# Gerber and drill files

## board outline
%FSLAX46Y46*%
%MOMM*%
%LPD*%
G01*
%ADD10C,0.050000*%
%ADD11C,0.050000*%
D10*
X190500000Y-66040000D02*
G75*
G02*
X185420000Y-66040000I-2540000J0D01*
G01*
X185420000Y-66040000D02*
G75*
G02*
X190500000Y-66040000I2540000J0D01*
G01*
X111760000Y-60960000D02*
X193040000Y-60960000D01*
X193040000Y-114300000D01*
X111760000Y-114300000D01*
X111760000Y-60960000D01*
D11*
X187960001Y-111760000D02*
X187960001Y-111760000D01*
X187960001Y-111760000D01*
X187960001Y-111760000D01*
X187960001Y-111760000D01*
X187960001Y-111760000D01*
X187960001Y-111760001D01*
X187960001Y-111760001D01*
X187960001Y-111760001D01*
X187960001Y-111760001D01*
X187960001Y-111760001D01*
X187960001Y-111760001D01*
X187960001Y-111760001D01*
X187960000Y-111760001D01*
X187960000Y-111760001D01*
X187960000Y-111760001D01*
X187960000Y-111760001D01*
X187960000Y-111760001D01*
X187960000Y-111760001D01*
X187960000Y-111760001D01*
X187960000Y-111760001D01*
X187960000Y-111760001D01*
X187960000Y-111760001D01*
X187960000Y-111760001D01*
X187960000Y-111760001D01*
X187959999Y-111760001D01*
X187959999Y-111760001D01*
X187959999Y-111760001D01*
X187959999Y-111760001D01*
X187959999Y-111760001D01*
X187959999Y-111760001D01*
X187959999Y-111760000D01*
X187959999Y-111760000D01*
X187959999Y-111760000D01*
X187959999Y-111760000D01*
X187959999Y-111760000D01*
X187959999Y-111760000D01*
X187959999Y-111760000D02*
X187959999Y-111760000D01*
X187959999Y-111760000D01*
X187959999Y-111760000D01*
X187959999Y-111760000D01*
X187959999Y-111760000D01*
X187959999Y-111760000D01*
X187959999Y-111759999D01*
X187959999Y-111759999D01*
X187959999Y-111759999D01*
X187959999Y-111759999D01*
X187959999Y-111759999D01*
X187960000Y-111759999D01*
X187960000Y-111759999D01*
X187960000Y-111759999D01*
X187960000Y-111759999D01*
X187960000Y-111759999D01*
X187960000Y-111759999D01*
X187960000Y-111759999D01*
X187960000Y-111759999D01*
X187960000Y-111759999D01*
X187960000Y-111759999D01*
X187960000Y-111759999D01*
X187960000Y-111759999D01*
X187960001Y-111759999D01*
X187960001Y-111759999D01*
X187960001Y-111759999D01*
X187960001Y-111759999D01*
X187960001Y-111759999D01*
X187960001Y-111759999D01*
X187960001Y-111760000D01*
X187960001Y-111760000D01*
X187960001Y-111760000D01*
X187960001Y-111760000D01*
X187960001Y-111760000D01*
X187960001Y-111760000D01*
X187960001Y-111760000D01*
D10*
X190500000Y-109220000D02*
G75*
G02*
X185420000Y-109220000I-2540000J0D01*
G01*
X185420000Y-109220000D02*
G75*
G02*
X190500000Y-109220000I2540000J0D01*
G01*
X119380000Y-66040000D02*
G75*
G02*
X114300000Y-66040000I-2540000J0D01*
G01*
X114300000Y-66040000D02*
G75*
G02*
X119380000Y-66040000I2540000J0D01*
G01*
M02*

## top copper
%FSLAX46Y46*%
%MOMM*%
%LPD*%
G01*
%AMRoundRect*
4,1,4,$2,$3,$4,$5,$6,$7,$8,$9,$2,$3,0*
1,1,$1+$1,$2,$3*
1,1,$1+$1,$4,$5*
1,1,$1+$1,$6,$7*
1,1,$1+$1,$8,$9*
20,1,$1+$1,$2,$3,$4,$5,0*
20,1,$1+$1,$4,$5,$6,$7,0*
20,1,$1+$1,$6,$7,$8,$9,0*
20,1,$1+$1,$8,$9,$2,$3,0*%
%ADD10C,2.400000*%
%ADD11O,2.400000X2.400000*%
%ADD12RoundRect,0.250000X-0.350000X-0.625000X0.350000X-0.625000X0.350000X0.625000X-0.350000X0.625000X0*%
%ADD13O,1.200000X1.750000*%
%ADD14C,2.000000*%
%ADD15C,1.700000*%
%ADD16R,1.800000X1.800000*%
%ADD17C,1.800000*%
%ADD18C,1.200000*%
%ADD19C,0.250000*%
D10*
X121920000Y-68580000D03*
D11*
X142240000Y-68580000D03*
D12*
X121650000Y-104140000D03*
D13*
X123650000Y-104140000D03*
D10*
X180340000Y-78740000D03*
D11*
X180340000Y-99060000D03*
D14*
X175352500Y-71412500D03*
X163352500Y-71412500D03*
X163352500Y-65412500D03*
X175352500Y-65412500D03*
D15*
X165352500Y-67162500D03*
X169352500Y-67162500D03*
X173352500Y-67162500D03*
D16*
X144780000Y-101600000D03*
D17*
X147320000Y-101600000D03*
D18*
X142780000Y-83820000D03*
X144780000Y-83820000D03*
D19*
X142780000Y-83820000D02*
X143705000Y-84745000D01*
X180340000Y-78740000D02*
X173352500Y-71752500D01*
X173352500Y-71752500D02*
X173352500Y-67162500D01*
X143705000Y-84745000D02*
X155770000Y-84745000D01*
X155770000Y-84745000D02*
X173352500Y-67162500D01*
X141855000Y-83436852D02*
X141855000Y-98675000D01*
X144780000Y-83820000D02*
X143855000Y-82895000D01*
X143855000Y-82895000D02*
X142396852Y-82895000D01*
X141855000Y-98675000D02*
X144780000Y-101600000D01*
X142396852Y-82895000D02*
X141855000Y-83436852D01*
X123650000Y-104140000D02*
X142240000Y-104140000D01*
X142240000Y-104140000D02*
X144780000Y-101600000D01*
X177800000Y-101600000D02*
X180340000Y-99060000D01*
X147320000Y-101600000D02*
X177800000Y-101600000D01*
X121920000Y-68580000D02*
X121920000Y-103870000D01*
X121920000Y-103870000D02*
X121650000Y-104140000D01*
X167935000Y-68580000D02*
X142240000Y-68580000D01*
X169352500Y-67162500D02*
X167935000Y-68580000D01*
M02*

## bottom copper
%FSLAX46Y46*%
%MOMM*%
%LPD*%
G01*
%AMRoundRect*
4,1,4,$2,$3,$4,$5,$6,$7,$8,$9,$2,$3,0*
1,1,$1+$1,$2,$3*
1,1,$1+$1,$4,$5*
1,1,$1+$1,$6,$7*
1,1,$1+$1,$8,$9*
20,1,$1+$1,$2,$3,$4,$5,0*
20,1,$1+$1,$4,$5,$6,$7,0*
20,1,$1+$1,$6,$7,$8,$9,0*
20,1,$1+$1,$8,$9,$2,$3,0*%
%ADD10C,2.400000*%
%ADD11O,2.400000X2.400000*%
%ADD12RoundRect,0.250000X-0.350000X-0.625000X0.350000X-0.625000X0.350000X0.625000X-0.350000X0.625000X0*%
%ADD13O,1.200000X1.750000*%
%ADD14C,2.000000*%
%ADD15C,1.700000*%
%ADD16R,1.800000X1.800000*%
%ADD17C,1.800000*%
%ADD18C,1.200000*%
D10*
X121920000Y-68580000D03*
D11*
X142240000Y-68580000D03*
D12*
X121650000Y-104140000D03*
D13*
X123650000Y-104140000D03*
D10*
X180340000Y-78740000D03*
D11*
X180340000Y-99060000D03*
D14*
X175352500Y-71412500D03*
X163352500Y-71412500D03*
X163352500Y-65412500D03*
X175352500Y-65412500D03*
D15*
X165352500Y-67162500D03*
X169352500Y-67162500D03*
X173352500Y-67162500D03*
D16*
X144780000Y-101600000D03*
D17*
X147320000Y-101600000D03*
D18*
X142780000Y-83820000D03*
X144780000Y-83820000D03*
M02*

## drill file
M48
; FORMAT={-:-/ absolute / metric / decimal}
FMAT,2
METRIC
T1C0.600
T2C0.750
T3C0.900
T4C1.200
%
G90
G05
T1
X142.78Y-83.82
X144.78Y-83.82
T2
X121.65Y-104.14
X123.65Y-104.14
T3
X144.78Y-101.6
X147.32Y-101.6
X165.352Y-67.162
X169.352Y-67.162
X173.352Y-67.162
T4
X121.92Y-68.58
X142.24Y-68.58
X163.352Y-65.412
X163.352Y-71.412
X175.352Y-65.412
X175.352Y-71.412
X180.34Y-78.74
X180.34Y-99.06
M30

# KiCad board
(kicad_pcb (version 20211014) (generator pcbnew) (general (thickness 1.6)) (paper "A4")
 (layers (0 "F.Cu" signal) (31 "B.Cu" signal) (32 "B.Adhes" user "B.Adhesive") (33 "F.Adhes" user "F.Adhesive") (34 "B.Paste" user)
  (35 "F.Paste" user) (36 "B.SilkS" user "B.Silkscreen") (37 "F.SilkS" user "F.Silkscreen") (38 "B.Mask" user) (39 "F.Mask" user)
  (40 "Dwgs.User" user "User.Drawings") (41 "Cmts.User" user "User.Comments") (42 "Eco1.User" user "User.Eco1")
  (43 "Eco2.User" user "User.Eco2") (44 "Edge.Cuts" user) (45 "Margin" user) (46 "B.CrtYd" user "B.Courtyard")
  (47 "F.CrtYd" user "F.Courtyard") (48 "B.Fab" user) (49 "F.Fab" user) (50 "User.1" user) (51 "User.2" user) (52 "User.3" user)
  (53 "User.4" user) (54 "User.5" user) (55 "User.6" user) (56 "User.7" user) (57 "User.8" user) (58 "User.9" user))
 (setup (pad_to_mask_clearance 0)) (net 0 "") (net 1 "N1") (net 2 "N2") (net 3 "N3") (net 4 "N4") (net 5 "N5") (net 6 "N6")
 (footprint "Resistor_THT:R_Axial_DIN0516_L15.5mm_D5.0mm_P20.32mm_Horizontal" (layer "F.Cu") (at 121.92 68.58)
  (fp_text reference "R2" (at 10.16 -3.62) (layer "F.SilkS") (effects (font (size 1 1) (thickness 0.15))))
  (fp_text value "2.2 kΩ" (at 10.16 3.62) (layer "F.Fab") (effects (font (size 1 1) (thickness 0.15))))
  (pad "1" thru_hole circle (at 0 0) (size 2.4 2.4) (drill 1.2) (layers *.Cu *.Mask) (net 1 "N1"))
  (pad "2" thru_hole oval (at 20.32 0) (size 2.4 2.4) (drill 1.2) (layers *.Cu *.Mask) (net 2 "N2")))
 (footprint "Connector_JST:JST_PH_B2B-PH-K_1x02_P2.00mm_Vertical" (layer "F.Cu") (at 121.65 104.14)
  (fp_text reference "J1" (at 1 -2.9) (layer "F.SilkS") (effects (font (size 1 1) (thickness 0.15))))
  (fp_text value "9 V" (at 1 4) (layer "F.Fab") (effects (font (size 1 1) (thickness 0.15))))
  (pad "1" thru_hole roundrect (at 0 0) (size 1.2 1.75) (drill 0.75) (layers *.Cu *.Mask) (roundrect_rratio 0.208333) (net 1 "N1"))
  (pad "2" thru_hole oval (at 2 0) (size 1.2 1.75) (drill 0.75) (layers *.Cu *.Mask) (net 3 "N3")))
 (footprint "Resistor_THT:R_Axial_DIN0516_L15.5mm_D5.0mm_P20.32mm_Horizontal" (layer "F.Cu") (at 180.34 78.74 -90)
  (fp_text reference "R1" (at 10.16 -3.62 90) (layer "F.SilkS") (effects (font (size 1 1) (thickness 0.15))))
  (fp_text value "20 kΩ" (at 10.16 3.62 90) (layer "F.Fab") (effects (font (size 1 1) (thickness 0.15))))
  (pad "1" thru_hole circle (at 0 0 270) (size 2.4 2.4) (drill 1.2) (layers *.Cu *.Mask) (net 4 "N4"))
  (pad "2" thru_hole oval (at 20.32 0 270) (size 2.4 2.4) (drill 1.2) (layers *.Cu *.Mask) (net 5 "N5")))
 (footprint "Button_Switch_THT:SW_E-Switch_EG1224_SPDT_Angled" (layer "F.Cu") (at 165.3525 67.1625)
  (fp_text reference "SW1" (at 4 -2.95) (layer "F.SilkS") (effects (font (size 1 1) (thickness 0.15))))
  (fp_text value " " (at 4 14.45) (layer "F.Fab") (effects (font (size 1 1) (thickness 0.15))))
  (pad "" thru_hole circle (at 10 4.25) (size 2 2) (drill 1.2) (layers *.Cu *.Mask))
  (pad "" thru_hole circle (at -2 4.25) (size 2 2) (drill 1.2) (layers *.Cu *.Mask))
  (pad "" thru_hole circle (at -2 -1.75) (size 2 2) (drill 1.2) (layers *.Cu *.Mask))
  (pad "" thru_hole circle (at 10 -1.75) (size 2 2) (drill 1.2) (layers *.Cu *.Mask))
  (pad "1" thru_hole circle (at 0 0) (size 1.7 1.7) (drill 0.9) (layers *.Cu *.Mask) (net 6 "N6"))
  (pad "2" thru_hole circle (at 4 0) (size 1.7 1.7) (drill 0.9) (layers *.Cu *.Mask) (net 2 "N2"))
  (pad "3" thru_hole circle (at 8 0) (size 1.7 1.7) (drill 0.9) (layers *.Cu *.Mask) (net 4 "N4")))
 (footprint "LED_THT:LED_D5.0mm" (layer "F.Cu") (at 144.78 101.6)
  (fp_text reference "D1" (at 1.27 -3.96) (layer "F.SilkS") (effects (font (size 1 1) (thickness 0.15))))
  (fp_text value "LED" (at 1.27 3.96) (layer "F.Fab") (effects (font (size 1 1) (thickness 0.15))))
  (pad "1" thru_hole rect (at 0 0) (size 1.8 1.8) (drill 0.9) (layers *.Cu *.Mask) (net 3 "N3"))
  (pad "2" thru_hole circle (at 2.54 0) (size 1.8 1.8) (drill 0.9) (layers *.Cu *.Mask) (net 5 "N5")))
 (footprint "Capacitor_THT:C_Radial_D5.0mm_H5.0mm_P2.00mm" (layer "F.Cu") (at 142.78 83.82)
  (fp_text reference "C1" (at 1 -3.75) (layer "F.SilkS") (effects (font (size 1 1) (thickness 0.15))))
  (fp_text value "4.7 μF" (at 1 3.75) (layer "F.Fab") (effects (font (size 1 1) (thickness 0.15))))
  (pad "1" thru_hole circle (at 0 0) (size 1.2 1.2) (drill 0.6) (layers *.Cu *.Mask) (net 4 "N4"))
  (pad "2" thru_hole circle (at 2 0) (size 1.2 1.2) (drill 0.6) (layers *.Cu *.Mask) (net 3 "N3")))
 (gr_circle (center 187.96 66.04) (end 187.96 68.58) (layer "Edge.Cuts") (width 0.05) (fill none))
 (gr_rect (start 193.04 114.3) (end 111.76 60.96) (layer "Edge.Cuts") (width 0.05) (fill none))
 (gr_circle (center 187.96 111.76) (end 187.96 111.76) (layer "Edge.Cuts") (width 0.05) (fill none))
 (gr_circle (center 187.96 109.22) (end 187.96 111.76) (layer "Edge.Cuts") (width 0.05) (fill none))
 (gr_circle (center 116.84 66.04) (end 119.38 66.04) (layer "Edge.Cuts") (width 0.05) (fill none))
 (segment (start 142.78 83.82) (end 143.705 84.745) (width 0.25) (layer "F.Cu") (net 4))
 (segment (start 180.34 78.74) (end 173.3525 71.7525) (width 0.25) (layer "F.Cu") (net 4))
 (segment (start 173.3525 71.7525) (end 173.3525 67.1625) (width 0.25) (layer "F.Cu") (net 4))
 (segment (start 143.705 84.745) (end 155.77 84.745) (width 0.25) (layer "F.Cu") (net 4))
 (segment (start 155.77 84.745) (end 173.3525 67.1625) (width 0.25) (layer "F.Cu") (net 4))
 (segment (start 141.855 83.436852) (end 141.855 98.675) (width 0.25) (layer "F.Cu") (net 3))
 (segment (start 144.78 83.82) (end 143.855 82.895) (width 0.25) (layer "F.Cu") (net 3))
 (segment (start 143.855 82.895) (end 142.396852 82.895) (width 0.25) (layer "F.Cu") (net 3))
 (segment (start 141.855 98.675) (end 144.78 101.6) (width 0.25) (layer "F.Cu") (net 3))
 (segment (start 142.396852 82.895) (end 141.855 83.436852) (width 0.25) (layer "F.Cu") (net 3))
 (segment (start 123.65 104.14) (end 142.24 104.14) (width 0.25) (layer "F.Cu") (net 3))
 (segment (start 142.24 104.14) (end 144.78 101.6) (width 0.25) (layer "F.Cu") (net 3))
 (segment (start 177.8 101.6) (end 180.34 99.06) (width 0.25) (layer "F.Cu") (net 5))
 (segment (start 147.32 101.6) (end 177.8 101.6) (width 0.25) (layer "F.Cu") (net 5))
 (segment (start 121.92 68.58) (end 121.92 103.87) (width 0.25) (layer "F.Cu") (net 1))
 (segment (start 121.92 103.87) (end 121.65 104.14) (width 0.25) (layer "F.Cu") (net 1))
 (segment (start 167.935 68.58) (end 142.24 68.58) (width 0.25) (layer "F.Cu") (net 2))
 (segment (start 169.3525 67.1625) (end 167.935 68.58) (width 0.25) (layer "F.Cu") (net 2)))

